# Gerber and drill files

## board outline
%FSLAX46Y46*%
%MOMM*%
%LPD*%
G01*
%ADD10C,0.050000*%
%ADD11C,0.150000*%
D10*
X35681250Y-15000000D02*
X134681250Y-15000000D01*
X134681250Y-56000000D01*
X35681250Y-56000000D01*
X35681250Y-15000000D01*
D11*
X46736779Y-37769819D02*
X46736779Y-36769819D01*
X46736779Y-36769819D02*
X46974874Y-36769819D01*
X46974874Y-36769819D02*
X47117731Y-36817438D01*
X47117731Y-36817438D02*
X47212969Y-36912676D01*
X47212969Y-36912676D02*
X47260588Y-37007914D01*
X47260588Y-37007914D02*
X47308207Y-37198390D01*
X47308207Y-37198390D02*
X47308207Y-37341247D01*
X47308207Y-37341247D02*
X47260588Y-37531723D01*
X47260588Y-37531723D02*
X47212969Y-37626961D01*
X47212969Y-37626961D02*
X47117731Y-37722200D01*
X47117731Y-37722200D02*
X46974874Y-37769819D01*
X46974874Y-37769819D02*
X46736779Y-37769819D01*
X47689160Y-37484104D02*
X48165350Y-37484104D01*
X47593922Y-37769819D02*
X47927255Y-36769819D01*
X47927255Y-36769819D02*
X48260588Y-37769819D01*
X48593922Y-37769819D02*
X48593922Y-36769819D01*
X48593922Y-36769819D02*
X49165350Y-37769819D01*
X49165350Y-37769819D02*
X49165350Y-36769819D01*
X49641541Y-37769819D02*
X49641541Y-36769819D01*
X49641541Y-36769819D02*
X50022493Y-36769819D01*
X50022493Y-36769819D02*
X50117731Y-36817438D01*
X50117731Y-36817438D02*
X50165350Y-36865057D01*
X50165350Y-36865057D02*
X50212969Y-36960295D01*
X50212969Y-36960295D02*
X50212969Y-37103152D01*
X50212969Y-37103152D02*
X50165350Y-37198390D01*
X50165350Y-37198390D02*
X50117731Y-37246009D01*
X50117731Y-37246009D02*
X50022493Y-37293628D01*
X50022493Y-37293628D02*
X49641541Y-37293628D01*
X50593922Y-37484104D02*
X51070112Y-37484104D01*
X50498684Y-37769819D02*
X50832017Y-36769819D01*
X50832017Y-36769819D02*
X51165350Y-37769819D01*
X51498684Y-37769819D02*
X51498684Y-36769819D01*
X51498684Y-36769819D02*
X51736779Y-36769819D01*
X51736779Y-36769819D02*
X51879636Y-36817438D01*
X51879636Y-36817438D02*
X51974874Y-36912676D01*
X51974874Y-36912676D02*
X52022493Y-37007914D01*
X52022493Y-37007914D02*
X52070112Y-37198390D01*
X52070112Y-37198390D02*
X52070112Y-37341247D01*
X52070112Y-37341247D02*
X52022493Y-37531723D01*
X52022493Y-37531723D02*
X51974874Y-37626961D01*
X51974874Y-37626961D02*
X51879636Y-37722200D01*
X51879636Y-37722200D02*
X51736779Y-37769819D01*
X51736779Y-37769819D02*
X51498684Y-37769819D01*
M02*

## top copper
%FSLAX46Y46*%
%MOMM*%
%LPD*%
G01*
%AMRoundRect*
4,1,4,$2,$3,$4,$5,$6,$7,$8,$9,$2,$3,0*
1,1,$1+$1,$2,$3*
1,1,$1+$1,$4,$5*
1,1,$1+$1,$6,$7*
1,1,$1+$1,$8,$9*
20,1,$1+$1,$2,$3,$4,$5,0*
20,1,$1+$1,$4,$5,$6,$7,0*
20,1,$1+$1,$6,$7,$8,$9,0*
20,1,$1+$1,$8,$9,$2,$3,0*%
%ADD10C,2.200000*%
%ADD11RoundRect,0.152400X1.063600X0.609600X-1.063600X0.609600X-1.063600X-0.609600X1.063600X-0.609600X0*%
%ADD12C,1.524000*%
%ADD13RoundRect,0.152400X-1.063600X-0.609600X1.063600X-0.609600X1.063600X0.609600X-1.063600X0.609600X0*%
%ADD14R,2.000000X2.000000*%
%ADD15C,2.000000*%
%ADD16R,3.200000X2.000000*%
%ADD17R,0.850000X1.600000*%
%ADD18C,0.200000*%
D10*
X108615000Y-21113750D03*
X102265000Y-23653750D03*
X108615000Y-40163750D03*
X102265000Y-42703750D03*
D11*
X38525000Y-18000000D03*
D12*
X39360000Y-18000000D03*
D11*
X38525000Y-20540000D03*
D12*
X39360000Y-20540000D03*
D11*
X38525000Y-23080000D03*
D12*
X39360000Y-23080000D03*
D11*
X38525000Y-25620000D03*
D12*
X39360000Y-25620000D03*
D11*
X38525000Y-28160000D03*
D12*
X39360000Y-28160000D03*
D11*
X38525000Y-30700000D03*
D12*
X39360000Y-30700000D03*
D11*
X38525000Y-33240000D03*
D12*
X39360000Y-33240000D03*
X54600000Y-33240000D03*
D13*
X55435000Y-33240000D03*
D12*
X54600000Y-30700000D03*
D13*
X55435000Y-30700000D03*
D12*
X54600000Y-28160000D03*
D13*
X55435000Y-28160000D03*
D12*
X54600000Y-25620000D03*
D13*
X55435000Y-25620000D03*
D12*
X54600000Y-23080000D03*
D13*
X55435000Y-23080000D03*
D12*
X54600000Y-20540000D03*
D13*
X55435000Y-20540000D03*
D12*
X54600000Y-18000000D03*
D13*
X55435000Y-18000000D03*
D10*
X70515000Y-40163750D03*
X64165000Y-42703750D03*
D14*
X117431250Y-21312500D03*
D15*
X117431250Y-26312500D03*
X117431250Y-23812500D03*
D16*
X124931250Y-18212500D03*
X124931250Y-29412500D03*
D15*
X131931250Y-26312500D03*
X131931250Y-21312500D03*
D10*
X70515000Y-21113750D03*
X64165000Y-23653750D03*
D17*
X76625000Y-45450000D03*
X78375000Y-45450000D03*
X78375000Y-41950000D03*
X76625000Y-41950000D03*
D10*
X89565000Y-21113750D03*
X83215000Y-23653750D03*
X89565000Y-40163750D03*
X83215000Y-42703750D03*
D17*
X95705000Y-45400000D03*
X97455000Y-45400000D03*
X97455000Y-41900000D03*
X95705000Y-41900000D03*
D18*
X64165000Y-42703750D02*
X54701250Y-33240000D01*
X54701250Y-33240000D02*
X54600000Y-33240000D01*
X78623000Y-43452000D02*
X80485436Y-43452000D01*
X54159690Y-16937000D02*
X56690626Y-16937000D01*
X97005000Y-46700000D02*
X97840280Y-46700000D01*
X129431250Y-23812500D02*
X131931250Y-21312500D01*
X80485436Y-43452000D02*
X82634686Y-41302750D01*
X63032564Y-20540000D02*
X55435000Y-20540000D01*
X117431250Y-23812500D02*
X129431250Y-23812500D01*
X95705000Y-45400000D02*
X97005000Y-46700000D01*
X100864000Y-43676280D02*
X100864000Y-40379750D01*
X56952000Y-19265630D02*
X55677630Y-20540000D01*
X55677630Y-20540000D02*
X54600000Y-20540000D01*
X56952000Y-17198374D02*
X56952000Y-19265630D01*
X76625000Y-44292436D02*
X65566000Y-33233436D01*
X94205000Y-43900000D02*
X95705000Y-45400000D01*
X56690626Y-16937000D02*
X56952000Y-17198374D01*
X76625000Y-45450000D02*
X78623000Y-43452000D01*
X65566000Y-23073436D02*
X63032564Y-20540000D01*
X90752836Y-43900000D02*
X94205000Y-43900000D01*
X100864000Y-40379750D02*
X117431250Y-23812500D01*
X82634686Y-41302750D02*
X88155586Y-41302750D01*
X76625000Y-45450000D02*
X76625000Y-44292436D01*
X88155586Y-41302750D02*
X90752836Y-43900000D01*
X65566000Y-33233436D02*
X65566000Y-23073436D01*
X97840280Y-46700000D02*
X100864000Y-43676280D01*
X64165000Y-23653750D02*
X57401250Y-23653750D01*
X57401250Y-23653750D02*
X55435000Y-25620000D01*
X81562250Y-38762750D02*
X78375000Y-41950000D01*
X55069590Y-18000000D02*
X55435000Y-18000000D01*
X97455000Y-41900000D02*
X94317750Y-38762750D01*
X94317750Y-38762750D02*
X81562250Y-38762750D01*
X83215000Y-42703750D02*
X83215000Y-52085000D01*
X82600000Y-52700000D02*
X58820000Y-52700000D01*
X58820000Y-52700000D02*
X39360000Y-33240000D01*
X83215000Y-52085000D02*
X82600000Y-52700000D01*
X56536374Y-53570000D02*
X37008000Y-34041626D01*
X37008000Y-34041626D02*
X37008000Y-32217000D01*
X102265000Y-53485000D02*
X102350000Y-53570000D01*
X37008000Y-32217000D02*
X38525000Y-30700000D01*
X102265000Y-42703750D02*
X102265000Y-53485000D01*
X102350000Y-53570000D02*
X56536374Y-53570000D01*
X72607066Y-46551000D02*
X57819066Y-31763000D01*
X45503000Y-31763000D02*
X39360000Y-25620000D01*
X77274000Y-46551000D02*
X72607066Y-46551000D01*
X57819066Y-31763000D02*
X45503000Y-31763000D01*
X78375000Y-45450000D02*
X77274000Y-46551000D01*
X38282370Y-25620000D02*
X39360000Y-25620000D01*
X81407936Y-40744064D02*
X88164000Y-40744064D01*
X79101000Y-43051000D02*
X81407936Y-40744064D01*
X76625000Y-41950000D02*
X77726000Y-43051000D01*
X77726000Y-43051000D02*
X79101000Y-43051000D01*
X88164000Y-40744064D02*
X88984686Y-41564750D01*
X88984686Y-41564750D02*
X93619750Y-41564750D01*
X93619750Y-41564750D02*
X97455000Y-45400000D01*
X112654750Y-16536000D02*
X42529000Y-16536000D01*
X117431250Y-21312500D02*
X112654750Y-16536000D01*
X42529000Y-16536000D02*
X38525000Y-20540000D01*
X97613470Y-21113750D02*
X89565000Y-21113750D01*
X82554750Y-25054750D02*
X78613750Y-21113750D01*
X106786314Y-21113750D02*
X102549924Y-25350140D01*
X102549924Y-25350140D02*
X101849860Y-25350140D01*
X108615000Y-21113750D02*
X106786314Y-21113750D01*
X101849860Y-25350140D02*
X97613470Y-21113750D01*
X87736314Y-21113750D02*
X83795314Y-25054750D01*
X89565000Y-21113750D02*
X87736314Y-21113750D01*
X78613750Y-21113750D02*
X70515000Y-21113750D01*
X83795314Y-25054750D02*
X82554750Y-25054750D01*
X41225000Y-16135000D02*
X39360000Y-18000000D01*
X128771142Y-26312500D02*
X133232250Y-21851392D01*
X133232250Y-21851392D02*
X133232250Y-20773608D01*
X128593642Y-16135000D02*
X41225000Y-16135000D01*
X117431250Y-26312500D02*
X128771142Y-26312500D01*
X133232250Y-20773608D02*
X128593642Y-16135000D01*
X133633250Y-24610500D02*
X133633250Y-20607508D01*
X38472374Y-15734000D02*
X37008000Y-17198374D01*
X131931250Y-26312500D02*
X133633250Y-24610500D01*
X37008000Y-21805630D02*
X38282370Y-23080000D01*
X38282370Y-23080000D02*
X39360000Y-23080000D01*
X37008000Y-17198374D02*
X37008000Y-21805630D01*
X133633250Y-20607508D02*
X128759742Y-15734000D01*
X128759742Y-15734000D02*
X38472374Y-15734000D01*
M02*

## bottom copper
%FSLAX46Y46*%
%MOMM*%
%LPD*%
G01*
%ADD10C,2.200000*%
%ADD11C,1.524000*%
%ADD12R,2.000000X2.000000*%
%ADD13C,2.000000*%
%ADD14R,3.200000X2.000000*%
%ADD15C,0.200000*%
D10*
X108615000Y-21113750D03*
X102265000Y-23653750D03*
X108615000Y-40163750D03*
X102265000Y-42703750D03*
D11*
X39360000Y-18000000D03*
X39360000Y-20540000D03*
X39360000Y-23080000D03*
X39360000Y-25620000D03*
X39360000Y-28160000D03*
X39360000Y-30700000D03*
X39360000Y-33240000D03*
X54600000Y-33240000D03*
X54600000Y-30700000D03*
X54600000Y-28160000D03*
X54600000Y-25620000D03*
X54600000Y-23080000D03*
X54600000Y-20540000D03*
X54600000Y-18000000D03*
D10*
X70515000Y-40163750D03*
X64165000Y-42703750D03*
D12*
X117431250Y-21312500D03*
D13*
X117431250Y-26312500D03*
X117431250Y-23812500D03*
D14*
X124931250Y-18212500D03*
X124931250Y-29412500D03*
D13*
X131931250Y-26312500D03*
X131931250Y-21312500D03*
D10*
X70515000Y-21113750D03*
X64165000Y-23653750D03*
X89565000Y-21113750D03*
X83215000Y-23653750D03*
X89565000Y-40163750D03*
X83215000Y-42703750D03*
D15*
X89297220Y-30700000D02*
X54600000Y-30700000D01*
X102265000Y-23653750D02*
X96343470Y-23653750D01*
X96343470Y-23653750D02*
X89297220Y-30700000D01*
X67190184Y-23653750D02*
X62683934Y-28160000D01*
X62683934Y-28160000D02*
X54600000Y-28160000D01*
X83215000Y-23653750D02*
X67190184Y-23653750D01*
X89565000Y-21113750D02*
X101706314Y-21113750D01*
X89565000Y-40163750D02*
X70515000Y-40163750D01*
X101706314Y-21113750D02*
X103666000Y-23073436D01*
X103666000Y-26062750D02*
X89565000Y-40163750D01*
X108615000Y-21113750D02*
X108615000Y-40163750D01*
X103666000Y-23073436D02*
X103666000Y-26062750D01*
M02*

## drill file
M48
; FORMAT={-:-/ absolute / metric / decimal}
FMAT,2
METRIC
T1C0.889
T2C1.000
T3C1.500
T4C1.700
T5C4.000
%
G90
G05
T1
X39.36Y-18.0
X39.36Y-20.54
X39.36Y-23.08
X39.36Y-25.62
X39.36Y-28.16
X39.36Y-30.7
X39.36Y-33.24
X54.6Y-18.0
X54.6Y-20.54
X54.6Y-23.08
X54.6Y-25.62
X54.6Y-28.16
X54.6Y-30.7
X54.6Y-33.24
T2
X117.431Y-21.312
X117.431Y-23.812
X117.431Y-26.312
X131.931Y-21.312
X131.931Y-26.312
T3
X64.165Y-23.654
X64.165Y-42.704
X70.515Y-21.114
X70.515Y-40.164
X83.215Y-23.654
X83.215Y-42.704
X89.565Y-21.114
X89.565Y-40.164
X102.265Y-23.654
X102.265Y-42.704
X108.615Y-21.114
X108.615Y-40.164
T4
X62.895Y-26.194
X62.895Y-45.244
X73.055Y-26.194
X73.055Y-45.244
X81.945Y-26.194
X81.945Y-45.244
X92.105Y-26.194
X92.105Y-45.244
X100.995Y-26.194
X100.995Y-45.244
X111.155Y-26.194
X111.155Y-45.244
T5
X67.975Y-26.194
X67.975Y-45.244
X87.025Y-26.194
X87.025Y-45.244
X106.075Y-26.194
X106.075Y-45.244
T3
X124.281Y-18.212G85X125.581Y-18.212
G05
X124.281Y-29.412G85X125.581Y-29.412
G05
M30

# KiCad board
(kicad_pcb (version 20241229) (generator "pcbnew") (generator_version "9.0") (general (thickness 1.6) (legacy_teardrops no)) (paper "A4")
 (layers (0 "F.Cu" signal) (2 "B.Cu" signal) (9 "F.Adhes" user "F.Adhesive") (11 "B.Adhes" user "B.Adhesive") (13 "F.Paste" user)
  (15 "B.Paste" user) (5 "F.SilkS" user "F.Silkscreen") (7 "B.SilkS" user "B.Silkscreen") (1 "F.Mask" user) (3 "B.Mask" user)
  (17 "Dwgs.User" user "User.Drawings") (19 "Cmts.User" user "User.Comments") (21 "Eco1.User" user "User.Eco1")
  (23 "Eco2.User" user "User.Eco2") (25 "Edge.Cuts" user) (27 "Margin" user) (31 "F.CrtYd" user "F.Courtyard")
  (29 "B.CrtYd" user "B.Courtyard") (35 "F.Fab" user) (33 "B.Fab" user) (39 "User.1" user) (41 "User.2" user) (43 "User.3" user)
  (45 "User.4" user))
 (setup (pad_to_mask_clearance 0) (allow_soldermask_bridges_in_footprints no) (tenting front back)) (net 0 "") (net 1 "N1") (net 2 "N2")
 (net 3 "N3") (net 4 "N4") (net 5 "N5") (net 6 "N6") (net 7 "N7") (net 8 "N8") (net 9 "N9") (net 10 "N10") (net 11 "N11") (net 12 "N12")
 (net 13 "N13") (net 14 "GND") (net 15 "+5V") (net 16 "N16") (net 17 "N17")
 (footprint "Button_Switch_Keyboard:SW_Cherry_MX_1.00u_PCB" (layer "F.Cu") (at 108.615 21.11375)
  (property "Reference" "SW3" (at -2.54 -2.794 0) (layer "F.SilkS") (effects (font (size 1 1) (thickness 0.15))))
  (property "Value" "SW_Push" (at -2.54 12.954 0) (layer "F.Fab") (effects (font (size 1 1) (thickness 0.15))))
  (pad "" np_thru_hole circle (at -7.62 5.08) (size 1.7 1.7) (drill 1.7) (layers "*.Cu" "*.Mask"))
  (pad "" np_thru_hole circle (at -2.54 5.08) (size 4 4) (drill 4) (layers "*.Cu" "*.Mask"))
  (pad "" np_thru_hole circle (at 2.54 5.08) (size 1.7 1.7) (drill 1.7) (layers "*.Cu" "*.Mask"))
  (pad "1" thru_hole circle (at 0 0) (size 2.2 2.2) (drill 1.5) (layers "*.Cu" "*.Mask") (remove_unused_layers no) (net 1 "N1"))
  (pad "2" thru_hole circle (at -6.35 2.54) (size 2.2 2.2) (drill 1.5) (layers "*.Cu" "*.Mask") (remove_unused_layers no) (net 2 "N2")))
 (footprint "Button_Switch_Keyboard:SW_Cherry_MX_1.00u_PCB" (layer "F.Cu") (at 108.615 40.16375)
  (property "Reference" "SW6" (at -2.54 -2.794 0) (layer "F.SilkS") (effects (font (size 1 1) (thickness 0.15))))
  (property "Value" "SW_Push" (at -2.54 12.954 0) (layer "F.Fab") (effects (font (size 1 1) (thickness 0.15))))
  (pad "" np_thru_hole circle (at -7.62 5.08) (size 1.7 1.7) (drill 1.7) (layers "*.Cu" "*.Mask"))
  (pad "" np_thru_hole circle (at -2.54 5.08) (size 4 4) (drill 4) (layers "*.Cu" "*.Mask"))
  (pad "" np_thru_hole circle (at 2.54 5.08) (size 1.7 1.7) (drill 1.7) (layers "*.Cu" "*.Mask"))
  (pad "1" thru_hole circle (at 0 0) (size 2.2 2.2) (drill 1.5) (layers "*.Cu" "*.Mask") (remove_unused_layers no) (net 1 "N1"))
  (pad "2" thru_hole circle (at -6.35 2.54) (size 2.2 2.2) (drill 1.5) (layers "*.Cu" "*.Mask") (remove_unused_layers no) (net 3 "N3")))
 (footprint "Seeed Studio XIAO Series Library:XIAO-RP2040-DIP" (layer "F.Cu") (at 46.98 25.62)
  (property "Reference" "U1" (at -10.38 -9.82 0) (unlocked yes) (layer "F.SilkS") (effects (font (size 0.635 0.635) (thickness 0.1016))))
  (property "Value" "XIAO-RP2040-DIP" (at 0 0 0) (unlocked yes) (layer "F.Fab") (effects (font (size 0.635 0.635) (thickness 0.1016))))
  (pad "1" smd roundrect (at -8.455 -7.62 180) (size 2.432 1.524) (layers "F.Cu" "F.Mask") (roundrect_rratio 0.1) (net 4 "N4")
   (thermal_bridge_angle 45))
  (pad "1" thru_hole circle (at -7.62 -7.62 180) (size 1.524 1.524) (drill 0.889) (layers "*.Cu" "*.Mask") (remove_unused_layers no)
   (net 4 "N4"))
  (pad "2" smd roundrect (at -8.455 -5.08 180) (size 2.432 1.524) (layers "F.Cu" "F.Mask") (roundrect_rratio 0.1) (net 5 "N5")
   (thermal_bridge_angle 45))
  (pad "2" thru_hole circle (at -7.62 -5.08 180) (size 1.524 1.524) (drill 0.889) (layers "*.Cu" "*.Mask") (remove_unused_layers no)
   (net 5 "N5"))
  (pad "3" smd roundrect (at -8.455 -2.54 180) (size 2.432 1.524) (layers "F.Cu" "F.Mask") (roundrect_rratio 0.1) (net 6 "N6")
   (thermal_bridge_angle 45))
  (pad "3" thru_hole circle (at -7.62 -2.54 180) (size 1.524 1.524) (drill 0.889) (layers "*.Cu" "*.Mask") (remove_unused_layers no)
   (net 6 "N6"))
  (pad "4" smd roundrect (at -8.455 0 180) (size 2.432 1.524) (layers "F.Cu" "F.Mask") (roundrect_rratio 0.1) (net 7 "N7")
   (thermal_bridge_angle 45))
  (pad "4" thru_hole circle (at -7.62 0 180) (size 1.524 1.524) (drill 0.889) (layers "*.Cu" "*.Mask") (remove_unused_layers no)
   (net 7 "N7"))
  (pad "5" smd roundrect (at -8.455 2.54 180) (size 2.432 1.524) (layers "F.Cu" "F.Mask") (roundrect_rratio 0.1) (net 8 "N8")
   (thermal_bridge_angle 45))
  (pad "5" thru_hole circle (at -7.62 2.54 180) (size 1.524 1.524) (drill 0.889) (layers "*.Cu" "*.Mask") (remove_unused_layers no)
   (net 8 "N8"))
  (pad "6" smd roundrect (at -8.455 5.08 180) (size 2.432 1.524) (layers "F.Cu" "F.Mask") (roundrect_rratio 0.1) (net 3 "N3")
   (thermal_bridge_angle 45))
  (pad "6" thru_hole circle (at -7.62 5.08 180) (size 1.524 1.524) (drill 0.889) (layers "*.Cu" "*.Mask") (remove_unused_layers no)
   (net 3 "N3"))
  (pad "7" smd roundrect (at -8.455 7.62 180) (size 2.432 1.524) (layers "F.Cu" "F.Mask") (roundrect_rratio 0.1) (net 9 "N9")
   (thermal_bridge_angle 45))
  (pad "7" thru_hole circle (at -7.62 7.62 180) (size 1.524 1.524) (drill 0.889) (layers "*.Cu" "*.Mask") (remove_unused_layers no)
   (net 9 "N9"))
  (pad "8" thru_hole circle (at 7.62 7.62) (size 1.524 1.524) (drill 0.889) (layers "*.Cu" "*.Mask") (remove_unused_layers no)
   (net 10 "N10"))
  (pad "8" smd roundrect (at 8.455 7.62) (size 2.432 1.524) (layers "F.Cu" "F.Mask") (roundrect_rratio 0.1) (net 10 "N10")
   (thermal_bridge_angle 45))
  (pad "9" thru_hole circle (at 7.62 5.08) (size 1.524 1.524) (drill 0.889) (layers "*.Cu" "*.Mask") (remove_unused_layers no) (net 2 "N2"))
  (pad "9" smd roundrect (at 8.455 5.08) (size 2.432 1.524) (layers "F.Cu" "F.Mask") (roundrect_rratio 0.1) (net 2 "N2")
   (thermal_bridge_angle 45))
  (pad "10" thru_hole circle (at 7.62 2.54) (size 1.524 1.524) (drill 0.889) (layers "*.Cu" "*.Mask") (remove_unused_layers no)
   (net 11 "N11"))
  (pad "10" smd roundrect (at 8.455 2.54) (size 2.432 1.524) (layers "F.Cu" "F.Mask") (roundrect_rratio 0.1) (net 11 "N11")
   (thermal_bridge_angle 45))
  (pad "11" thru_hole circle (at 7.62 0) (size 1.524 1.524) (drill 0.889) (layers "*.Cu" "*.Mask") (remove_unused_layers no) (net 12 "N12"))
  (pad "11" smd roundrect (at 8.455 0) (size 2.432 1.524) (layers "F.Cu" "F.Mask") (roundrect_rratio 0.1) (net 12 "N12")
   (thermal_bridge_angle 45))
  (pad "12" thru_hole circle (at 7.62 -2.54) (size 1.524 1.524) (drill 0.889) (layers "*.Cu" "*.Mask") (remove_unused_layers no)
   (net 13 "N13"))
  (pad "12" smd roundrect (at 8.455 -2.54) (size 2.432 1.524) (layers "F.Cu" "F.Mask") (roundrect_rratio 0.1) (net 13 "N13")
   (thermal_bridge_angle 45))
  (pad "13" thru_hole circle (at 7.62 -5.08) (size 1.524 1.524) (drill 0.889) (layers "*.Cu" "*.Mask") (remove_unused_layers no)
   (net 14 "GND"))
  (pad "13" smd roundrect (at 8.455 -5.08) (size 2.432 1.524) (layers "F.Cu" "F.Mask") (roundrect_rratio 0.1) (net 14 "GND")
   (thermal_bridge_angle 45))
  (pad "14" thru_hole circle (at 7.62 -7.62) (size 1.524 1.524) (drill 0.889) (layers "*.Cu" "*.Mask") (remove_unused_layers no)
   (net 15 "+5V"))
  (pad "14" smd roundrect (at 8.455 -7.62) (size 2.432 1.524) (layers "F.Cu" "F.Mask") (roundrect_rratio 0.1) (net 15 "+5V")
   (thermal_bridge_angle 45)))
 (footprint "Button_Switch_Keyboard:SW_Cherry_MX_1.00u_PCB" (layer "F.Cu") (at 70.515 40.16375)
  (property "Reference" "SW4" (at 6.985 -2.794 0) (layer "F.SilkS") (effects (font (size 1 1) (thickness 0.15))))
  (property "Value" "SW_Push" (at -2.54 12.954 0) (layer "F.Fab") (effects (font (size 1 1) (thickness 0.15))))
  (pad "" np_thru_hole circle (at -7.62 5.08) (size 1.7 1.7) (drill 1.7) (layers "*.Cu" "*.Mask"))
  (pad "" np_thru_hole circle (at -2.54 5.08) (size 4 4) (drill 4) (layers "*.Cu" "*.Mask"))
  (pad "" np_thru_hole circle (at 2.54 5.08) (size 1.7 1.7) (drill 1.7) (layers "*.Cu" "*.Mask"))
  (pad "1" thru_hole circle (at 0 0) (size 2.2 2.2) (drill 1.5) (layers "*.Cu" "*.Mask") (remove_unused_layers no) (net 1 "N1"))
  (pad "2" thru_hole circle (at -6.35 2.54) (size 2.2 2.2) (drill 1.5) (layers "*.Cu" "*.Mask") (remove_unused_layers no) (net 10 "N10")))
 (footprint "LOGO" (layer "F.Cu") (at 45.6 43.5)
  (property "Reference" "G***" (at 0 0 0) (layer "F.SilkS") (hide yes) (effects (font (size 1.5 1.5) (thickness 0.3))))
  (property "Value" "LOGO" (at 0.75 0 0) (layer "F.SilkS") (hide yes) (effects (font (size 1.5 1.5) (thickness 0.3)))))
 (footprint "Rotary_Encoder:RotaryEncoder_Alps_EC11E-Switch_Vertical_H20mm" (layer "F.Cu") (at 117.43125 21.3125)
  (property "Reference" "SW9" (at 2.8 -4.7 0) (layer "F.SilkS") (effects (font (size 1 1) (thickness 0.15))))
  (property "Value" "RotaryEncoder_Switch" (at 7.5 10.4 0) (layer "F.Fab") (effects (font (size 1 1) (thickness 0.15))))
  (pad "A" thru_hole rect (at 0 0) (size 2 2) (drill 1) (layers "*.Cu" "*.Mask") (remove_unused_layers no) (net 5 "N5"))
  (pad "B" thru_hole circle (at 0 5) (size 2 2) (drill 1) (layers "*.Cu" "*.Mask") (remove_unused_layers no) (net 4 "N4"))
  (pad "C" thru_hole circle (at 0 2.5) (size 2 2) (drill 1) (layers "*.Cu" "*.Mask") (remove_unused_layers no) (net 14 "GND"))
  (pad "MP" thru_hole rect (at 7.5 -3.1) (size 3.2 2) (drill oval 2.8 1.5) (layers "*.Cu" "*.Mask") (remove_unused_layers no))
  (pad "MP" thru_hole rect (at 7.5 8.1) (size 3.2 2) (drill oval 2.8 1.5) (layers "*.Cu" "*.Mask") (remove_unused_layers no))
  (pad "S1" thru_hole circle (at 14.5 5) (size 2 2) (drill 1) (layers "*.Cu" "*.Mask") (remove_unused_layers no) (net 6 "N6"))
  (pad "S2" thru_hole circle (at 14.5 0) (size 2 2) (drill 1) (layers "*.Cu" "*.Mask") (remove_unused_layers no) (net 14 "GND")))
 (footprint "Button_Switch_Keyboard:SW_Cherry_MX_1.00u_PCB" (layer "F.Cu") (at 70.515 21.11375)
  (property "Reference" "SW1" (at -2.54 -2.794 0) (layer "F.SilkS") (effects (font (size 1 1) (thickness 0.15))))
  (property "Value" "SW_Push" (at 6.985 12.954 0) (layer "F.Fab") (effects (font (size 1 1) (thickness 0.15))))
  (pad "" np_thru_hole circle (at -7.62 5.08) (size 1.7 1.7) (drill 1.7) (layers "*.Cu" "*.Mask"))
  (pad "" np_thru_hole circle (at -2.54 5.08) (size 4 4) (drill 4) (layers "*.Cu" "*.Mask"))
  (pad "" np_thru_hole circle (at 2.54 5.08) (size 1.7 1.7) (drill 1.7) (layers "*.Cu" "*.Mask"))
  (pad "1" thru_hole circle (at 0 0) (size 2.2 2.2) (drill 1.5) (layers "*.Cu" "*.Mask") (remove_unused_layers no) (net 1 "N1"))
  (pad "2" thru_hole circle (at -6.35 2.54) (size 2.2 2.2) (drill 1.5) (layers "*.Cu" "*.Mask") (remove_unused_layers no) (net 12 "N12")))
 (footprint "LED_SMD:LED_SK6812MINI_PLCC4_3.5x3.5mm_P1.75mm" (layer "F.Cu") (at 77.5 43.7 90)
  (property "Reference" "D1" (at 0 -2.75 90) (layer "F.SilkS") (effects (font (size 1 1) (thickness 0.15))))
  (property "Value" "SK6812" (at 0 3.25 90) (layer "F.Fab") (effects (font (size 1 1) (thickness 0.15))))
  (pad "1" smd rect (at -1.75 -0.875 90) (size 1.6 0.85) (layers "F.Cu" "F.Mask" "F.Paste") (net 14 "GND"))
  (pad "2" smd rect (at -1.75 0.875 90) (size 1.6 0.85) (layers "F.Cu" "F.Mask" "F.Paste") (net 7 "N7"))
  (pad "3" smd rect (at 1.75 0.875 90) (size 1.6 0.85) (layers "F.Cu" "F.Mask" "F.Paste") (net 15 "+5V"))
  (pad "4" smd rect (at 1.75 -0.875 90) (size 1.6 0.85) (layers "F.Cu" "F.Mask" "F.Paste") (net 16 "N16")))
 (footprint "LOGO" (layer "F.Cu") (at 124.669887 44.700344)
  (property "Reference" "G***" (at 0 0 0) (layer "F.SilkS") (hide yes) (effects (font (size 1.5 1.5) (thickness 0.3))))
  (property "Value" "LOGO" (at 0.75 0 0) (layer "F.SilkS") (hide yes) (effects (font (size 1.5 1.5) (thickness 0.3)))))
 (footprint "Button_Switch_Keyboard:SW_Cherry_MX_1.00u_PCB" (layer "F.Cu") (at 89.565 21.11375)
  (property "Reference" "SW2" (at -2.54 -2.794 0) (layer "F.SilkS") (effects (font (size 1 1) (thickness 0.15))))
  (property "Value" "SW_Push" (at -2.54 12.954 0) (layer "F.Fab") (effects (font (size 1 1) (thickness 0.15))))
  (pad "" np_thru_hole circle (at -7.62 5.08) (size 1.7 1.7) (drill 1.7) (layers "*.Cu" "*.Mask"))
  (pad "" np_thru_hole circle (at -2.54 5.08) (size 4 4) (drill 4) (layers "*.Cu" "*.Mask"))
  (pad "" np_thru_hole circle (at 2.54 5.08) (size 1.7 1.7) (drill 1.7) (layers "*.Cu" "*.Mask"))
  (pad "1" thru_hole circle (at 0 0) (size 2.2 2.2) (drill 1.5) (layers "*.Cu" "*.Mask") (remove_unused_layers no) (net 1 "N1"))
  (pad "2" thru_hole circle (at -6.35 2.54) (size 2.2 2.2) (drill 1.5) (layers "*.Cu" "*.Mask") (remove_unused_layers no) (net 11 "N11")))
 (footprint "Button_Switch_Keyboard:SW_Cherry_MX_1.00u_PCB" (layer "F.Cu") (at 89.565 40.16375)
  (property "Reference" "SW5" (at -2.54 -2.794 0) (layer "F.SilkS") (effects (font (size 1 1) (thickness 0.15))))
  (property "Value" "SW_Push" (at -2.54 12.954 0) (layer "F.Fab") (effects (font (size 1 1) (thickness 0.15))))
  (pad "" np_thru_hole circle (at -7.62 5.08) (size 1.7 1.7) (drill 1.7) (layers "*.Cu" "*.Mask"))
  (pad "" np_thru_hole circle (at -2.54 5.08) (size 4 4) (drill 4) (layers "*.Cu" "*.Mask"))
  (pad "" np_thru_hole circle (at 2.54 5.08) (size 1.7 1.7) (drill 1.7) (layers "*.Cu" "*.Mask"))
  (pad "1" thru_hole circle (at 0 0) (size 2.2 2.2) (drill 1.5) (layers "*.Cu" "*.Mask") (remove_unused_layers no) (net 1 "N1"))
  (pad "2" thru_hole circle (at -6.35 2.54) (size 2.2 2.2) (drill 1.5) (layers "*.Cu" "*.Mask") (remove_unused_layers no) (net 9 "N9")))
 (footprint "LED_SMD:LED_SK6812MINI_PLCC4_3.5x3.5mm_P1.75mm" (layer "F.Cu") (at 96.58 43.65 90)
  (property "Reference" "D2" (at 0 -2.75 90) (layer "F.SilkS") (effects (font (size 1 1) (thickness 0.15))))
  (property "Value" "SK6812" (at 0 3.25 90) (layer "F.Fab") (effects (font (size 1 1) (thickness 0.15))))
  (pad "1" smd rect (at -1.75 -0.875 90) (size 1.6 0.85) (layers "F.Cu" "F.Mask" "F.Paste") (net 14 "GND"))
  (pad "2" smd rect (at -1.75 0.875 90) (size 1.6 0.85) (layers "F.Cu" "F.Mask" "F.Paste") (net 16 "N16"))
  (pad "3" smd rect (at 1.75 0.875 90) (size 1.6 0.85) (layers "F.Cu" "F.Mask" "F.Paste") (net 15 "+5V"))
  (pad "4" smd rect (at 1.75 -0.875 90) (size 1.6 0.85) (layers "F.Cu" "F.Mask" "F.Paste") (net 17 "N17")))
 (gr_rect (start 35.68125 15) (end 134.68125 56) (stroke (width 0.05) (type default)) (fill no) (layer "Edge.Cuts"))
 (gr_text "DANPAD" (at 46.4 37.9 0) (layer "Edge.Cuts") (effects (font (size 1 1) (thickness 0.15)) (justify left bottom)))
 (segment (start 64.165 42.70375) (end 54.70125 33.24) (width 0.2) (layer "F.Cu") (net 10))
 (segment (start 54.70125 33.24) (end 54.6 33.24) (width 0.2) (layer "F.Cu") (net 10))
 (segment (start 78.623 43.452) (end 80.485436 43.452) (width 0.2) (layer "F.Cu") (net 14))
 (segment (start 54.15969 16.937) (end 56.690626 16.937) (width 0.2) (layer "F.Cu") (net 14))
 (segment (start 97.005 46.7) (end 97.84028 46.7) (width 0.2) (layer "F.Cu") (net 14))
 (segment (start 129.43125 23.8125) (end 131.93125 21.3125) (width 0.2) (layer "F.Cu") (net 14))
 (segment (start 80.485436 43.452) (end 82.634686 41.30275) (width 0.2) (layer "F.Cu") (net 14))
 (segment (start 63.032564 20.54) (end 55.435 20.54) (width 0.2) (layer "F.Cu") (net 14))
 (segment (start 117.43125 23.8125) (end 129.43125 23.8125) (width 0.2) (layer "F.Cu") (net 14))
 (segment (start 95.705 45.4) (end 97.005 46.7) (width 0.2) (layer "F.Cu") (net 14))
 (segment (start 100.864 43.67628) (end 100.864 40.37975) (width 0.2) (layer "F.Cu") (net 14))
 (segment (start 56.952 19.26563) (end 55.67763 20.54) (width 0.2) (layer "F.Cu") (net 14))
 (segment (start 55.67763 20.54) (end 54.6 20.54) (width 0.2) (layer "F.Cu") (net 14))
 (segment (start 56.952 17.198374) (end 56.952 19.26563) (width 0.2) (layer "F.Cu") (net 14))
 (segment (start 76.625 44.292436) (end 65.566 33.233436) (width 0.2) (layer "F.Cu") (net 14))
 (segment (start 94.205 43.9) (end 95.705 45.4) (width 0.2) (layer "F.Cu") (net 14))
 (segment (start 56.690626 16.937) (end 56.952 17.198374) (width 0.2) (layer "F.Cu") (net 14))
 (segment (start 76.625 45.45) (end 78.623 43.452) (width 0.2) (layer "F.Cu") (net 14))
 (segment (start 65.566 23.073436) (end 63.032564 20.54) (width 0.2) (layer "F.Cu") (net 14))
 (segment (start 90.752836 43.9) (end 94.205 43.9) (width 0.2) (layer "F.Cu") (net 14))
 (segment (start 100.864 40.37975) (end 117.43125 23.8125) (width 0.2) (layer "F.Cu") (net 14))
 (segment (start 82.634686 41.30275) (end 88.155586 41.30275) (width 0.2) (layer "F.Cu") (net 14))
 (segment (start 76.625 45.45) (end 76.625 44.292436) (width 0.2) (layer "F.Cu") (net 14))
 (segment (start 88.155586 41.30275) (end 90.752836 43.9) (width 0.2) (layer "F.Cu") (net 14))
 (segment (start 65.566 33.233436) (end 65.566 23.073436) (width 0.2) (layer "F.Cu") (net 14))
 (segment (start 97.84028 46.7) (end 100.864 43.67628) (width 0.2) (layer "F.Cu") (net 14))
 (segment (start 89.29722 30.7) (end 54.6 30.7) (width 0.2) (layer "B.Cu") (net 2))
 (segment (start 102.265 23.65375) (end 96.34347 23.65375) (width 0.2) (layer "B.Cu") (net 2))
 (segment (start 96.34347 23.65375) (end 89.29722 30.7) (width 0.2) (layer "B.Cu") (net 2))
 (segment (start 67.190184 23.65375) (end 62.683934 28.16) (width 0.2) (layer "B.Cu") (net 11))
 (segment (start 62.683934 28.16) (end 54.6 28.16) (width 0.2) (layer "B.Cu") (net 11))
 (segment (start 83.215 23.65375) (end 67.190184 23.65375) (width 0.2) (layer "B.Cu") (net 11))
 (segment (start 64.165 23.65375) (end 57.40125 23.65375) (width 0.2) (layer "F.Cu") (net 12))
 (segment (start 57.40125 23.65375) (end 55.435 25.62) (width 0.2) (layer "F.Cu") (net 12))
 (segment (start 81.56225 38.76275) (end 78.375 41.95) (width 0.2) (layer "F.Cu") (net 15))
 (segment (start 55.06959 18) (end 55.435 18) (width 0.2) (layer "F.Cu") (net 15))
 (segment (start 97.455 41.9) (end 94.31775 38.76275) (width 0.2) (layer "F.Cu") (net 15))
 (segment (start 94.31775 38.76275) (end 81.56225 38.76275) (width 0.2) (layer "F.Cu") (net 15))
 (segment (start 83.215 42.70375) (end 83.215 52.085) (width 0.2) (layer "F.Cu") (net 9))
 (segment (start 82.6 52.7) (end 58.82 52.7) (width 0.2) (layer "F.Cu") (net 9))
 (segment (start 58.82 52.7) (end 39.36 33.24) (width 0.2) (layer "F.Cu") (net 9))
 (segment (start 83.215 52.085) (end 82.6 52.7) (width 0.2) (layer "F.Cu") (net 9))
 (segment (start 56.536374 53.57) (end 37.008 34.041626) (width 0.2) (layer "F.Cu") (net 3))
 (segment (start 37.008 34.041626) (end 37.008 32.217) (width 0.2) (layer "F.Cu") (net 3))
 (segment (start 102.265 53.485) (end 102.35 53.57) (width 0.2) (layer "F.Cu") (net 3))
 (segment (start 37.008 32.217) (end 38.525 30.7) (width 0.2) (layer "F.Cu") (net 3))
 (segment (start 102.265 42.70375) (end 102.265 53.485) (width 0.2) (layer "F.Cu") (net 3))
 (segment (start 102.35 53.57) (end 56.536374 53.57) (width 0.2) (layer "F.Cu") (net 3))
 (segment (start 72.607066 46.551) (end 57.819066 31.763) (width 0.2) (layer "F.Cu") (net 7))
 (segment (start 45.503 31.763) (end 39.36 25.62) (width 0.2) (layer "F.Cu") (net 7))
 (segment (start 77.274 46.551) (end 72.607066 46.551) (width 0.2) (layer "F.Cu") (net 7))
 (segment (start 57.819066 31.763) (end 45.503 31.763) (width 0.2) (layer "F.Cu") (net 7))
 (segment (start 78.375 45.45) (end 77.274 46.551) (width 0.2) (layer "F.Cu") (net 7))
 (segment (start 38.28237 25.62) (end 39.36 25.62) (width 0.2) (layer "F.Cu") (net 7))
 (segment (start 81.407936 40.744064) (end 88.164 40.744064) (width 0.2) (layer "F.Cu") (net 16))
 (segment (start 79.101 43.051) (end 81.407936 40.744064) (width 0.2) (layer "F.Cu") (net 16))
 (segment (start 76.625 41.95) (end 77.726 43.051) (width 0.2) (layer "F.Cu") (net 16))
 (segment (start 77.726 43.051) (end 79.101 43.051) (width 0.2) (layer "F.Cu") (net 16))
 (segment (start 88.164 40.744064) (end 88.984686 41.56475) (width 0.2) (layer "F.Cu") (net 16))
 (segment (start 88.984686 41.56475) (end 93.61975 41.56475) (width 0.2) (layer "F.Cu") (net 16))
 (segment (start 93.61975 41.56475) (end 97.455 45.4) (width 0.2) (layer "F.Cu") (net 16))
 (segment (start 112.65475 16.536) (end 42.529 16.536) (width 0.2) (layer "F.Cu") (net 5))
 (segment (start 117.43125 21.3125) (end 112.65475 16.536) (width 0.2) (layer "F.Cu") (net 5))
 (segment (start 42.529 16.536) (end 38.525 20.54) (width 0.2) (layer "F.Cu") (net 5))
 (segment (start 97.61347 21.11375) (end 89.565 21.11375) (width 0.2) (layer "F.Cu") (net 1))
 (segment (start 82.55475 25.05475) (end 78.61375 21.11375) (width 0.2) (layer "F.Cu") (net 1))
 (segment (start 106.786314 21.11375) (end 102.549924 25.35014) (width 0.2) (layer "F.Cu") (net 1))
 (segment (start 102.549924 25.35014) (end 101.84986 25.35014) (width 0.2) (layer "F.Cu") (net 1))
 (segment (start 108.615 21.11375) (end 106.786314 21.11375) (width 0.2) (layer "F.Cu") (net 1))
 (segment (start 101.84986 25.35014) (end 97.61347 21.11375) (width 0.2) (layer "F.Cu") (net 1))
 (segment (start 87.736314 21.11375) (end 83.795314 25.05475) (width 0.2) (layer "F.Cu") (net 1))
 (segment (start 89.565 21.11375) (end 87.736314 21.11375) (width 0.2) (layer "F.Cu") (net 1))
 (segment (start 78.61375 21.11375) (end 70.515 21.11375) (width 0.2) (layer "F.Cu") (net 1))
 (segment (start 83.795314 25.05475) (end 82.55475 25.05475) (width 0.2) (layer "F.Cu") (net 1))
 (segment (start 89.565 21.11375) (end 101.706314 21.11375) (width 0.2) (layer "B.Cu") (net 1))
 (segment (start 89.565 40.16375) (end 70.515 40.16375) (width 0.2) (layer "B.Cu") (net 1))
 (segment (start 101.706314 21.11375) (end 103.666 23.073436) (width 0.2) (layer "B.Cu") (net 1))
 (segment (start 103.666 26.06275) (end 89.565 40.16375) (width 0.2) (layer "B.Cu") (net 1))
 (segment (start 108.615 21.11375) (end 108.615 40.16375) (width 0.2) (layer "B.Cu") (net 1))
 (segment (start 103.666 23.073436) (end 103.666 26.06275) (width 0.2) (layer "B.Cu") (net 1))
 (segment (start 41.225 16.135) (end 39.36 18) (width 0.2) (layer "F.Cu") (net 4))
 (segment (start 128.771142 26.3125) (end 133.23225 21.851392) (width 0.2) (layer "F.Cu") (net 4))
 (segment (start 133.23225 21.851392) (end 133.23225 20.773608) (width 0.2) (layer "F.Cu") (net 4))
 (segment (start 128.593642 16.135) (end 41.225 16.135) (width 0.2) (layer "F.Cu") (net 4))
 (segment (start 117.43125 26.3125) (end 128.771142 26.3125) (width 0.2) (layer "F.Cu") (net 4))
 (segment (start 133.23225 20.773608) (end 128.593642 16.135) (width 0.2) (layer "F.Cu") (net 4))
 (segment (start 133.63325 24.6105) (end 133.63325 20.607508) (width 0.2) (layer "F.Cu") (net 6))
 (segment (start 38.472374 15.734) (end 37.008 17.198374) (width 0.2) (layer "F.Cu") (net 6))
 (segment (start 131.93125 26.3125) (end 133.63325 24.6105) (width 0.2) (layer "F.Cu") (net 6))
 (segment (start 37.008 21.80563) (end 38.28237 23.08) (width 0.2) (layer "F.Cu") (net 6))
 (segment (start 38.28237 23.08) (end 39.36 23.08) (width 0.2) (layer "F.Cu") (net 6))
 (segment (start 37.008 17.198374) (end 37.008 21.80563) (width 0.2) (layer "F.Cu") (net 6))
 (segment (start 133.63325 20.607508) (end 128.759742 15.734) (width 0.2) (layer "F.Cu") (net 6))
 (segment (start 128.759742 15.734) (end 38.472374 15.734) (width 0.2) (layer "F.Cu") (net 6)))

